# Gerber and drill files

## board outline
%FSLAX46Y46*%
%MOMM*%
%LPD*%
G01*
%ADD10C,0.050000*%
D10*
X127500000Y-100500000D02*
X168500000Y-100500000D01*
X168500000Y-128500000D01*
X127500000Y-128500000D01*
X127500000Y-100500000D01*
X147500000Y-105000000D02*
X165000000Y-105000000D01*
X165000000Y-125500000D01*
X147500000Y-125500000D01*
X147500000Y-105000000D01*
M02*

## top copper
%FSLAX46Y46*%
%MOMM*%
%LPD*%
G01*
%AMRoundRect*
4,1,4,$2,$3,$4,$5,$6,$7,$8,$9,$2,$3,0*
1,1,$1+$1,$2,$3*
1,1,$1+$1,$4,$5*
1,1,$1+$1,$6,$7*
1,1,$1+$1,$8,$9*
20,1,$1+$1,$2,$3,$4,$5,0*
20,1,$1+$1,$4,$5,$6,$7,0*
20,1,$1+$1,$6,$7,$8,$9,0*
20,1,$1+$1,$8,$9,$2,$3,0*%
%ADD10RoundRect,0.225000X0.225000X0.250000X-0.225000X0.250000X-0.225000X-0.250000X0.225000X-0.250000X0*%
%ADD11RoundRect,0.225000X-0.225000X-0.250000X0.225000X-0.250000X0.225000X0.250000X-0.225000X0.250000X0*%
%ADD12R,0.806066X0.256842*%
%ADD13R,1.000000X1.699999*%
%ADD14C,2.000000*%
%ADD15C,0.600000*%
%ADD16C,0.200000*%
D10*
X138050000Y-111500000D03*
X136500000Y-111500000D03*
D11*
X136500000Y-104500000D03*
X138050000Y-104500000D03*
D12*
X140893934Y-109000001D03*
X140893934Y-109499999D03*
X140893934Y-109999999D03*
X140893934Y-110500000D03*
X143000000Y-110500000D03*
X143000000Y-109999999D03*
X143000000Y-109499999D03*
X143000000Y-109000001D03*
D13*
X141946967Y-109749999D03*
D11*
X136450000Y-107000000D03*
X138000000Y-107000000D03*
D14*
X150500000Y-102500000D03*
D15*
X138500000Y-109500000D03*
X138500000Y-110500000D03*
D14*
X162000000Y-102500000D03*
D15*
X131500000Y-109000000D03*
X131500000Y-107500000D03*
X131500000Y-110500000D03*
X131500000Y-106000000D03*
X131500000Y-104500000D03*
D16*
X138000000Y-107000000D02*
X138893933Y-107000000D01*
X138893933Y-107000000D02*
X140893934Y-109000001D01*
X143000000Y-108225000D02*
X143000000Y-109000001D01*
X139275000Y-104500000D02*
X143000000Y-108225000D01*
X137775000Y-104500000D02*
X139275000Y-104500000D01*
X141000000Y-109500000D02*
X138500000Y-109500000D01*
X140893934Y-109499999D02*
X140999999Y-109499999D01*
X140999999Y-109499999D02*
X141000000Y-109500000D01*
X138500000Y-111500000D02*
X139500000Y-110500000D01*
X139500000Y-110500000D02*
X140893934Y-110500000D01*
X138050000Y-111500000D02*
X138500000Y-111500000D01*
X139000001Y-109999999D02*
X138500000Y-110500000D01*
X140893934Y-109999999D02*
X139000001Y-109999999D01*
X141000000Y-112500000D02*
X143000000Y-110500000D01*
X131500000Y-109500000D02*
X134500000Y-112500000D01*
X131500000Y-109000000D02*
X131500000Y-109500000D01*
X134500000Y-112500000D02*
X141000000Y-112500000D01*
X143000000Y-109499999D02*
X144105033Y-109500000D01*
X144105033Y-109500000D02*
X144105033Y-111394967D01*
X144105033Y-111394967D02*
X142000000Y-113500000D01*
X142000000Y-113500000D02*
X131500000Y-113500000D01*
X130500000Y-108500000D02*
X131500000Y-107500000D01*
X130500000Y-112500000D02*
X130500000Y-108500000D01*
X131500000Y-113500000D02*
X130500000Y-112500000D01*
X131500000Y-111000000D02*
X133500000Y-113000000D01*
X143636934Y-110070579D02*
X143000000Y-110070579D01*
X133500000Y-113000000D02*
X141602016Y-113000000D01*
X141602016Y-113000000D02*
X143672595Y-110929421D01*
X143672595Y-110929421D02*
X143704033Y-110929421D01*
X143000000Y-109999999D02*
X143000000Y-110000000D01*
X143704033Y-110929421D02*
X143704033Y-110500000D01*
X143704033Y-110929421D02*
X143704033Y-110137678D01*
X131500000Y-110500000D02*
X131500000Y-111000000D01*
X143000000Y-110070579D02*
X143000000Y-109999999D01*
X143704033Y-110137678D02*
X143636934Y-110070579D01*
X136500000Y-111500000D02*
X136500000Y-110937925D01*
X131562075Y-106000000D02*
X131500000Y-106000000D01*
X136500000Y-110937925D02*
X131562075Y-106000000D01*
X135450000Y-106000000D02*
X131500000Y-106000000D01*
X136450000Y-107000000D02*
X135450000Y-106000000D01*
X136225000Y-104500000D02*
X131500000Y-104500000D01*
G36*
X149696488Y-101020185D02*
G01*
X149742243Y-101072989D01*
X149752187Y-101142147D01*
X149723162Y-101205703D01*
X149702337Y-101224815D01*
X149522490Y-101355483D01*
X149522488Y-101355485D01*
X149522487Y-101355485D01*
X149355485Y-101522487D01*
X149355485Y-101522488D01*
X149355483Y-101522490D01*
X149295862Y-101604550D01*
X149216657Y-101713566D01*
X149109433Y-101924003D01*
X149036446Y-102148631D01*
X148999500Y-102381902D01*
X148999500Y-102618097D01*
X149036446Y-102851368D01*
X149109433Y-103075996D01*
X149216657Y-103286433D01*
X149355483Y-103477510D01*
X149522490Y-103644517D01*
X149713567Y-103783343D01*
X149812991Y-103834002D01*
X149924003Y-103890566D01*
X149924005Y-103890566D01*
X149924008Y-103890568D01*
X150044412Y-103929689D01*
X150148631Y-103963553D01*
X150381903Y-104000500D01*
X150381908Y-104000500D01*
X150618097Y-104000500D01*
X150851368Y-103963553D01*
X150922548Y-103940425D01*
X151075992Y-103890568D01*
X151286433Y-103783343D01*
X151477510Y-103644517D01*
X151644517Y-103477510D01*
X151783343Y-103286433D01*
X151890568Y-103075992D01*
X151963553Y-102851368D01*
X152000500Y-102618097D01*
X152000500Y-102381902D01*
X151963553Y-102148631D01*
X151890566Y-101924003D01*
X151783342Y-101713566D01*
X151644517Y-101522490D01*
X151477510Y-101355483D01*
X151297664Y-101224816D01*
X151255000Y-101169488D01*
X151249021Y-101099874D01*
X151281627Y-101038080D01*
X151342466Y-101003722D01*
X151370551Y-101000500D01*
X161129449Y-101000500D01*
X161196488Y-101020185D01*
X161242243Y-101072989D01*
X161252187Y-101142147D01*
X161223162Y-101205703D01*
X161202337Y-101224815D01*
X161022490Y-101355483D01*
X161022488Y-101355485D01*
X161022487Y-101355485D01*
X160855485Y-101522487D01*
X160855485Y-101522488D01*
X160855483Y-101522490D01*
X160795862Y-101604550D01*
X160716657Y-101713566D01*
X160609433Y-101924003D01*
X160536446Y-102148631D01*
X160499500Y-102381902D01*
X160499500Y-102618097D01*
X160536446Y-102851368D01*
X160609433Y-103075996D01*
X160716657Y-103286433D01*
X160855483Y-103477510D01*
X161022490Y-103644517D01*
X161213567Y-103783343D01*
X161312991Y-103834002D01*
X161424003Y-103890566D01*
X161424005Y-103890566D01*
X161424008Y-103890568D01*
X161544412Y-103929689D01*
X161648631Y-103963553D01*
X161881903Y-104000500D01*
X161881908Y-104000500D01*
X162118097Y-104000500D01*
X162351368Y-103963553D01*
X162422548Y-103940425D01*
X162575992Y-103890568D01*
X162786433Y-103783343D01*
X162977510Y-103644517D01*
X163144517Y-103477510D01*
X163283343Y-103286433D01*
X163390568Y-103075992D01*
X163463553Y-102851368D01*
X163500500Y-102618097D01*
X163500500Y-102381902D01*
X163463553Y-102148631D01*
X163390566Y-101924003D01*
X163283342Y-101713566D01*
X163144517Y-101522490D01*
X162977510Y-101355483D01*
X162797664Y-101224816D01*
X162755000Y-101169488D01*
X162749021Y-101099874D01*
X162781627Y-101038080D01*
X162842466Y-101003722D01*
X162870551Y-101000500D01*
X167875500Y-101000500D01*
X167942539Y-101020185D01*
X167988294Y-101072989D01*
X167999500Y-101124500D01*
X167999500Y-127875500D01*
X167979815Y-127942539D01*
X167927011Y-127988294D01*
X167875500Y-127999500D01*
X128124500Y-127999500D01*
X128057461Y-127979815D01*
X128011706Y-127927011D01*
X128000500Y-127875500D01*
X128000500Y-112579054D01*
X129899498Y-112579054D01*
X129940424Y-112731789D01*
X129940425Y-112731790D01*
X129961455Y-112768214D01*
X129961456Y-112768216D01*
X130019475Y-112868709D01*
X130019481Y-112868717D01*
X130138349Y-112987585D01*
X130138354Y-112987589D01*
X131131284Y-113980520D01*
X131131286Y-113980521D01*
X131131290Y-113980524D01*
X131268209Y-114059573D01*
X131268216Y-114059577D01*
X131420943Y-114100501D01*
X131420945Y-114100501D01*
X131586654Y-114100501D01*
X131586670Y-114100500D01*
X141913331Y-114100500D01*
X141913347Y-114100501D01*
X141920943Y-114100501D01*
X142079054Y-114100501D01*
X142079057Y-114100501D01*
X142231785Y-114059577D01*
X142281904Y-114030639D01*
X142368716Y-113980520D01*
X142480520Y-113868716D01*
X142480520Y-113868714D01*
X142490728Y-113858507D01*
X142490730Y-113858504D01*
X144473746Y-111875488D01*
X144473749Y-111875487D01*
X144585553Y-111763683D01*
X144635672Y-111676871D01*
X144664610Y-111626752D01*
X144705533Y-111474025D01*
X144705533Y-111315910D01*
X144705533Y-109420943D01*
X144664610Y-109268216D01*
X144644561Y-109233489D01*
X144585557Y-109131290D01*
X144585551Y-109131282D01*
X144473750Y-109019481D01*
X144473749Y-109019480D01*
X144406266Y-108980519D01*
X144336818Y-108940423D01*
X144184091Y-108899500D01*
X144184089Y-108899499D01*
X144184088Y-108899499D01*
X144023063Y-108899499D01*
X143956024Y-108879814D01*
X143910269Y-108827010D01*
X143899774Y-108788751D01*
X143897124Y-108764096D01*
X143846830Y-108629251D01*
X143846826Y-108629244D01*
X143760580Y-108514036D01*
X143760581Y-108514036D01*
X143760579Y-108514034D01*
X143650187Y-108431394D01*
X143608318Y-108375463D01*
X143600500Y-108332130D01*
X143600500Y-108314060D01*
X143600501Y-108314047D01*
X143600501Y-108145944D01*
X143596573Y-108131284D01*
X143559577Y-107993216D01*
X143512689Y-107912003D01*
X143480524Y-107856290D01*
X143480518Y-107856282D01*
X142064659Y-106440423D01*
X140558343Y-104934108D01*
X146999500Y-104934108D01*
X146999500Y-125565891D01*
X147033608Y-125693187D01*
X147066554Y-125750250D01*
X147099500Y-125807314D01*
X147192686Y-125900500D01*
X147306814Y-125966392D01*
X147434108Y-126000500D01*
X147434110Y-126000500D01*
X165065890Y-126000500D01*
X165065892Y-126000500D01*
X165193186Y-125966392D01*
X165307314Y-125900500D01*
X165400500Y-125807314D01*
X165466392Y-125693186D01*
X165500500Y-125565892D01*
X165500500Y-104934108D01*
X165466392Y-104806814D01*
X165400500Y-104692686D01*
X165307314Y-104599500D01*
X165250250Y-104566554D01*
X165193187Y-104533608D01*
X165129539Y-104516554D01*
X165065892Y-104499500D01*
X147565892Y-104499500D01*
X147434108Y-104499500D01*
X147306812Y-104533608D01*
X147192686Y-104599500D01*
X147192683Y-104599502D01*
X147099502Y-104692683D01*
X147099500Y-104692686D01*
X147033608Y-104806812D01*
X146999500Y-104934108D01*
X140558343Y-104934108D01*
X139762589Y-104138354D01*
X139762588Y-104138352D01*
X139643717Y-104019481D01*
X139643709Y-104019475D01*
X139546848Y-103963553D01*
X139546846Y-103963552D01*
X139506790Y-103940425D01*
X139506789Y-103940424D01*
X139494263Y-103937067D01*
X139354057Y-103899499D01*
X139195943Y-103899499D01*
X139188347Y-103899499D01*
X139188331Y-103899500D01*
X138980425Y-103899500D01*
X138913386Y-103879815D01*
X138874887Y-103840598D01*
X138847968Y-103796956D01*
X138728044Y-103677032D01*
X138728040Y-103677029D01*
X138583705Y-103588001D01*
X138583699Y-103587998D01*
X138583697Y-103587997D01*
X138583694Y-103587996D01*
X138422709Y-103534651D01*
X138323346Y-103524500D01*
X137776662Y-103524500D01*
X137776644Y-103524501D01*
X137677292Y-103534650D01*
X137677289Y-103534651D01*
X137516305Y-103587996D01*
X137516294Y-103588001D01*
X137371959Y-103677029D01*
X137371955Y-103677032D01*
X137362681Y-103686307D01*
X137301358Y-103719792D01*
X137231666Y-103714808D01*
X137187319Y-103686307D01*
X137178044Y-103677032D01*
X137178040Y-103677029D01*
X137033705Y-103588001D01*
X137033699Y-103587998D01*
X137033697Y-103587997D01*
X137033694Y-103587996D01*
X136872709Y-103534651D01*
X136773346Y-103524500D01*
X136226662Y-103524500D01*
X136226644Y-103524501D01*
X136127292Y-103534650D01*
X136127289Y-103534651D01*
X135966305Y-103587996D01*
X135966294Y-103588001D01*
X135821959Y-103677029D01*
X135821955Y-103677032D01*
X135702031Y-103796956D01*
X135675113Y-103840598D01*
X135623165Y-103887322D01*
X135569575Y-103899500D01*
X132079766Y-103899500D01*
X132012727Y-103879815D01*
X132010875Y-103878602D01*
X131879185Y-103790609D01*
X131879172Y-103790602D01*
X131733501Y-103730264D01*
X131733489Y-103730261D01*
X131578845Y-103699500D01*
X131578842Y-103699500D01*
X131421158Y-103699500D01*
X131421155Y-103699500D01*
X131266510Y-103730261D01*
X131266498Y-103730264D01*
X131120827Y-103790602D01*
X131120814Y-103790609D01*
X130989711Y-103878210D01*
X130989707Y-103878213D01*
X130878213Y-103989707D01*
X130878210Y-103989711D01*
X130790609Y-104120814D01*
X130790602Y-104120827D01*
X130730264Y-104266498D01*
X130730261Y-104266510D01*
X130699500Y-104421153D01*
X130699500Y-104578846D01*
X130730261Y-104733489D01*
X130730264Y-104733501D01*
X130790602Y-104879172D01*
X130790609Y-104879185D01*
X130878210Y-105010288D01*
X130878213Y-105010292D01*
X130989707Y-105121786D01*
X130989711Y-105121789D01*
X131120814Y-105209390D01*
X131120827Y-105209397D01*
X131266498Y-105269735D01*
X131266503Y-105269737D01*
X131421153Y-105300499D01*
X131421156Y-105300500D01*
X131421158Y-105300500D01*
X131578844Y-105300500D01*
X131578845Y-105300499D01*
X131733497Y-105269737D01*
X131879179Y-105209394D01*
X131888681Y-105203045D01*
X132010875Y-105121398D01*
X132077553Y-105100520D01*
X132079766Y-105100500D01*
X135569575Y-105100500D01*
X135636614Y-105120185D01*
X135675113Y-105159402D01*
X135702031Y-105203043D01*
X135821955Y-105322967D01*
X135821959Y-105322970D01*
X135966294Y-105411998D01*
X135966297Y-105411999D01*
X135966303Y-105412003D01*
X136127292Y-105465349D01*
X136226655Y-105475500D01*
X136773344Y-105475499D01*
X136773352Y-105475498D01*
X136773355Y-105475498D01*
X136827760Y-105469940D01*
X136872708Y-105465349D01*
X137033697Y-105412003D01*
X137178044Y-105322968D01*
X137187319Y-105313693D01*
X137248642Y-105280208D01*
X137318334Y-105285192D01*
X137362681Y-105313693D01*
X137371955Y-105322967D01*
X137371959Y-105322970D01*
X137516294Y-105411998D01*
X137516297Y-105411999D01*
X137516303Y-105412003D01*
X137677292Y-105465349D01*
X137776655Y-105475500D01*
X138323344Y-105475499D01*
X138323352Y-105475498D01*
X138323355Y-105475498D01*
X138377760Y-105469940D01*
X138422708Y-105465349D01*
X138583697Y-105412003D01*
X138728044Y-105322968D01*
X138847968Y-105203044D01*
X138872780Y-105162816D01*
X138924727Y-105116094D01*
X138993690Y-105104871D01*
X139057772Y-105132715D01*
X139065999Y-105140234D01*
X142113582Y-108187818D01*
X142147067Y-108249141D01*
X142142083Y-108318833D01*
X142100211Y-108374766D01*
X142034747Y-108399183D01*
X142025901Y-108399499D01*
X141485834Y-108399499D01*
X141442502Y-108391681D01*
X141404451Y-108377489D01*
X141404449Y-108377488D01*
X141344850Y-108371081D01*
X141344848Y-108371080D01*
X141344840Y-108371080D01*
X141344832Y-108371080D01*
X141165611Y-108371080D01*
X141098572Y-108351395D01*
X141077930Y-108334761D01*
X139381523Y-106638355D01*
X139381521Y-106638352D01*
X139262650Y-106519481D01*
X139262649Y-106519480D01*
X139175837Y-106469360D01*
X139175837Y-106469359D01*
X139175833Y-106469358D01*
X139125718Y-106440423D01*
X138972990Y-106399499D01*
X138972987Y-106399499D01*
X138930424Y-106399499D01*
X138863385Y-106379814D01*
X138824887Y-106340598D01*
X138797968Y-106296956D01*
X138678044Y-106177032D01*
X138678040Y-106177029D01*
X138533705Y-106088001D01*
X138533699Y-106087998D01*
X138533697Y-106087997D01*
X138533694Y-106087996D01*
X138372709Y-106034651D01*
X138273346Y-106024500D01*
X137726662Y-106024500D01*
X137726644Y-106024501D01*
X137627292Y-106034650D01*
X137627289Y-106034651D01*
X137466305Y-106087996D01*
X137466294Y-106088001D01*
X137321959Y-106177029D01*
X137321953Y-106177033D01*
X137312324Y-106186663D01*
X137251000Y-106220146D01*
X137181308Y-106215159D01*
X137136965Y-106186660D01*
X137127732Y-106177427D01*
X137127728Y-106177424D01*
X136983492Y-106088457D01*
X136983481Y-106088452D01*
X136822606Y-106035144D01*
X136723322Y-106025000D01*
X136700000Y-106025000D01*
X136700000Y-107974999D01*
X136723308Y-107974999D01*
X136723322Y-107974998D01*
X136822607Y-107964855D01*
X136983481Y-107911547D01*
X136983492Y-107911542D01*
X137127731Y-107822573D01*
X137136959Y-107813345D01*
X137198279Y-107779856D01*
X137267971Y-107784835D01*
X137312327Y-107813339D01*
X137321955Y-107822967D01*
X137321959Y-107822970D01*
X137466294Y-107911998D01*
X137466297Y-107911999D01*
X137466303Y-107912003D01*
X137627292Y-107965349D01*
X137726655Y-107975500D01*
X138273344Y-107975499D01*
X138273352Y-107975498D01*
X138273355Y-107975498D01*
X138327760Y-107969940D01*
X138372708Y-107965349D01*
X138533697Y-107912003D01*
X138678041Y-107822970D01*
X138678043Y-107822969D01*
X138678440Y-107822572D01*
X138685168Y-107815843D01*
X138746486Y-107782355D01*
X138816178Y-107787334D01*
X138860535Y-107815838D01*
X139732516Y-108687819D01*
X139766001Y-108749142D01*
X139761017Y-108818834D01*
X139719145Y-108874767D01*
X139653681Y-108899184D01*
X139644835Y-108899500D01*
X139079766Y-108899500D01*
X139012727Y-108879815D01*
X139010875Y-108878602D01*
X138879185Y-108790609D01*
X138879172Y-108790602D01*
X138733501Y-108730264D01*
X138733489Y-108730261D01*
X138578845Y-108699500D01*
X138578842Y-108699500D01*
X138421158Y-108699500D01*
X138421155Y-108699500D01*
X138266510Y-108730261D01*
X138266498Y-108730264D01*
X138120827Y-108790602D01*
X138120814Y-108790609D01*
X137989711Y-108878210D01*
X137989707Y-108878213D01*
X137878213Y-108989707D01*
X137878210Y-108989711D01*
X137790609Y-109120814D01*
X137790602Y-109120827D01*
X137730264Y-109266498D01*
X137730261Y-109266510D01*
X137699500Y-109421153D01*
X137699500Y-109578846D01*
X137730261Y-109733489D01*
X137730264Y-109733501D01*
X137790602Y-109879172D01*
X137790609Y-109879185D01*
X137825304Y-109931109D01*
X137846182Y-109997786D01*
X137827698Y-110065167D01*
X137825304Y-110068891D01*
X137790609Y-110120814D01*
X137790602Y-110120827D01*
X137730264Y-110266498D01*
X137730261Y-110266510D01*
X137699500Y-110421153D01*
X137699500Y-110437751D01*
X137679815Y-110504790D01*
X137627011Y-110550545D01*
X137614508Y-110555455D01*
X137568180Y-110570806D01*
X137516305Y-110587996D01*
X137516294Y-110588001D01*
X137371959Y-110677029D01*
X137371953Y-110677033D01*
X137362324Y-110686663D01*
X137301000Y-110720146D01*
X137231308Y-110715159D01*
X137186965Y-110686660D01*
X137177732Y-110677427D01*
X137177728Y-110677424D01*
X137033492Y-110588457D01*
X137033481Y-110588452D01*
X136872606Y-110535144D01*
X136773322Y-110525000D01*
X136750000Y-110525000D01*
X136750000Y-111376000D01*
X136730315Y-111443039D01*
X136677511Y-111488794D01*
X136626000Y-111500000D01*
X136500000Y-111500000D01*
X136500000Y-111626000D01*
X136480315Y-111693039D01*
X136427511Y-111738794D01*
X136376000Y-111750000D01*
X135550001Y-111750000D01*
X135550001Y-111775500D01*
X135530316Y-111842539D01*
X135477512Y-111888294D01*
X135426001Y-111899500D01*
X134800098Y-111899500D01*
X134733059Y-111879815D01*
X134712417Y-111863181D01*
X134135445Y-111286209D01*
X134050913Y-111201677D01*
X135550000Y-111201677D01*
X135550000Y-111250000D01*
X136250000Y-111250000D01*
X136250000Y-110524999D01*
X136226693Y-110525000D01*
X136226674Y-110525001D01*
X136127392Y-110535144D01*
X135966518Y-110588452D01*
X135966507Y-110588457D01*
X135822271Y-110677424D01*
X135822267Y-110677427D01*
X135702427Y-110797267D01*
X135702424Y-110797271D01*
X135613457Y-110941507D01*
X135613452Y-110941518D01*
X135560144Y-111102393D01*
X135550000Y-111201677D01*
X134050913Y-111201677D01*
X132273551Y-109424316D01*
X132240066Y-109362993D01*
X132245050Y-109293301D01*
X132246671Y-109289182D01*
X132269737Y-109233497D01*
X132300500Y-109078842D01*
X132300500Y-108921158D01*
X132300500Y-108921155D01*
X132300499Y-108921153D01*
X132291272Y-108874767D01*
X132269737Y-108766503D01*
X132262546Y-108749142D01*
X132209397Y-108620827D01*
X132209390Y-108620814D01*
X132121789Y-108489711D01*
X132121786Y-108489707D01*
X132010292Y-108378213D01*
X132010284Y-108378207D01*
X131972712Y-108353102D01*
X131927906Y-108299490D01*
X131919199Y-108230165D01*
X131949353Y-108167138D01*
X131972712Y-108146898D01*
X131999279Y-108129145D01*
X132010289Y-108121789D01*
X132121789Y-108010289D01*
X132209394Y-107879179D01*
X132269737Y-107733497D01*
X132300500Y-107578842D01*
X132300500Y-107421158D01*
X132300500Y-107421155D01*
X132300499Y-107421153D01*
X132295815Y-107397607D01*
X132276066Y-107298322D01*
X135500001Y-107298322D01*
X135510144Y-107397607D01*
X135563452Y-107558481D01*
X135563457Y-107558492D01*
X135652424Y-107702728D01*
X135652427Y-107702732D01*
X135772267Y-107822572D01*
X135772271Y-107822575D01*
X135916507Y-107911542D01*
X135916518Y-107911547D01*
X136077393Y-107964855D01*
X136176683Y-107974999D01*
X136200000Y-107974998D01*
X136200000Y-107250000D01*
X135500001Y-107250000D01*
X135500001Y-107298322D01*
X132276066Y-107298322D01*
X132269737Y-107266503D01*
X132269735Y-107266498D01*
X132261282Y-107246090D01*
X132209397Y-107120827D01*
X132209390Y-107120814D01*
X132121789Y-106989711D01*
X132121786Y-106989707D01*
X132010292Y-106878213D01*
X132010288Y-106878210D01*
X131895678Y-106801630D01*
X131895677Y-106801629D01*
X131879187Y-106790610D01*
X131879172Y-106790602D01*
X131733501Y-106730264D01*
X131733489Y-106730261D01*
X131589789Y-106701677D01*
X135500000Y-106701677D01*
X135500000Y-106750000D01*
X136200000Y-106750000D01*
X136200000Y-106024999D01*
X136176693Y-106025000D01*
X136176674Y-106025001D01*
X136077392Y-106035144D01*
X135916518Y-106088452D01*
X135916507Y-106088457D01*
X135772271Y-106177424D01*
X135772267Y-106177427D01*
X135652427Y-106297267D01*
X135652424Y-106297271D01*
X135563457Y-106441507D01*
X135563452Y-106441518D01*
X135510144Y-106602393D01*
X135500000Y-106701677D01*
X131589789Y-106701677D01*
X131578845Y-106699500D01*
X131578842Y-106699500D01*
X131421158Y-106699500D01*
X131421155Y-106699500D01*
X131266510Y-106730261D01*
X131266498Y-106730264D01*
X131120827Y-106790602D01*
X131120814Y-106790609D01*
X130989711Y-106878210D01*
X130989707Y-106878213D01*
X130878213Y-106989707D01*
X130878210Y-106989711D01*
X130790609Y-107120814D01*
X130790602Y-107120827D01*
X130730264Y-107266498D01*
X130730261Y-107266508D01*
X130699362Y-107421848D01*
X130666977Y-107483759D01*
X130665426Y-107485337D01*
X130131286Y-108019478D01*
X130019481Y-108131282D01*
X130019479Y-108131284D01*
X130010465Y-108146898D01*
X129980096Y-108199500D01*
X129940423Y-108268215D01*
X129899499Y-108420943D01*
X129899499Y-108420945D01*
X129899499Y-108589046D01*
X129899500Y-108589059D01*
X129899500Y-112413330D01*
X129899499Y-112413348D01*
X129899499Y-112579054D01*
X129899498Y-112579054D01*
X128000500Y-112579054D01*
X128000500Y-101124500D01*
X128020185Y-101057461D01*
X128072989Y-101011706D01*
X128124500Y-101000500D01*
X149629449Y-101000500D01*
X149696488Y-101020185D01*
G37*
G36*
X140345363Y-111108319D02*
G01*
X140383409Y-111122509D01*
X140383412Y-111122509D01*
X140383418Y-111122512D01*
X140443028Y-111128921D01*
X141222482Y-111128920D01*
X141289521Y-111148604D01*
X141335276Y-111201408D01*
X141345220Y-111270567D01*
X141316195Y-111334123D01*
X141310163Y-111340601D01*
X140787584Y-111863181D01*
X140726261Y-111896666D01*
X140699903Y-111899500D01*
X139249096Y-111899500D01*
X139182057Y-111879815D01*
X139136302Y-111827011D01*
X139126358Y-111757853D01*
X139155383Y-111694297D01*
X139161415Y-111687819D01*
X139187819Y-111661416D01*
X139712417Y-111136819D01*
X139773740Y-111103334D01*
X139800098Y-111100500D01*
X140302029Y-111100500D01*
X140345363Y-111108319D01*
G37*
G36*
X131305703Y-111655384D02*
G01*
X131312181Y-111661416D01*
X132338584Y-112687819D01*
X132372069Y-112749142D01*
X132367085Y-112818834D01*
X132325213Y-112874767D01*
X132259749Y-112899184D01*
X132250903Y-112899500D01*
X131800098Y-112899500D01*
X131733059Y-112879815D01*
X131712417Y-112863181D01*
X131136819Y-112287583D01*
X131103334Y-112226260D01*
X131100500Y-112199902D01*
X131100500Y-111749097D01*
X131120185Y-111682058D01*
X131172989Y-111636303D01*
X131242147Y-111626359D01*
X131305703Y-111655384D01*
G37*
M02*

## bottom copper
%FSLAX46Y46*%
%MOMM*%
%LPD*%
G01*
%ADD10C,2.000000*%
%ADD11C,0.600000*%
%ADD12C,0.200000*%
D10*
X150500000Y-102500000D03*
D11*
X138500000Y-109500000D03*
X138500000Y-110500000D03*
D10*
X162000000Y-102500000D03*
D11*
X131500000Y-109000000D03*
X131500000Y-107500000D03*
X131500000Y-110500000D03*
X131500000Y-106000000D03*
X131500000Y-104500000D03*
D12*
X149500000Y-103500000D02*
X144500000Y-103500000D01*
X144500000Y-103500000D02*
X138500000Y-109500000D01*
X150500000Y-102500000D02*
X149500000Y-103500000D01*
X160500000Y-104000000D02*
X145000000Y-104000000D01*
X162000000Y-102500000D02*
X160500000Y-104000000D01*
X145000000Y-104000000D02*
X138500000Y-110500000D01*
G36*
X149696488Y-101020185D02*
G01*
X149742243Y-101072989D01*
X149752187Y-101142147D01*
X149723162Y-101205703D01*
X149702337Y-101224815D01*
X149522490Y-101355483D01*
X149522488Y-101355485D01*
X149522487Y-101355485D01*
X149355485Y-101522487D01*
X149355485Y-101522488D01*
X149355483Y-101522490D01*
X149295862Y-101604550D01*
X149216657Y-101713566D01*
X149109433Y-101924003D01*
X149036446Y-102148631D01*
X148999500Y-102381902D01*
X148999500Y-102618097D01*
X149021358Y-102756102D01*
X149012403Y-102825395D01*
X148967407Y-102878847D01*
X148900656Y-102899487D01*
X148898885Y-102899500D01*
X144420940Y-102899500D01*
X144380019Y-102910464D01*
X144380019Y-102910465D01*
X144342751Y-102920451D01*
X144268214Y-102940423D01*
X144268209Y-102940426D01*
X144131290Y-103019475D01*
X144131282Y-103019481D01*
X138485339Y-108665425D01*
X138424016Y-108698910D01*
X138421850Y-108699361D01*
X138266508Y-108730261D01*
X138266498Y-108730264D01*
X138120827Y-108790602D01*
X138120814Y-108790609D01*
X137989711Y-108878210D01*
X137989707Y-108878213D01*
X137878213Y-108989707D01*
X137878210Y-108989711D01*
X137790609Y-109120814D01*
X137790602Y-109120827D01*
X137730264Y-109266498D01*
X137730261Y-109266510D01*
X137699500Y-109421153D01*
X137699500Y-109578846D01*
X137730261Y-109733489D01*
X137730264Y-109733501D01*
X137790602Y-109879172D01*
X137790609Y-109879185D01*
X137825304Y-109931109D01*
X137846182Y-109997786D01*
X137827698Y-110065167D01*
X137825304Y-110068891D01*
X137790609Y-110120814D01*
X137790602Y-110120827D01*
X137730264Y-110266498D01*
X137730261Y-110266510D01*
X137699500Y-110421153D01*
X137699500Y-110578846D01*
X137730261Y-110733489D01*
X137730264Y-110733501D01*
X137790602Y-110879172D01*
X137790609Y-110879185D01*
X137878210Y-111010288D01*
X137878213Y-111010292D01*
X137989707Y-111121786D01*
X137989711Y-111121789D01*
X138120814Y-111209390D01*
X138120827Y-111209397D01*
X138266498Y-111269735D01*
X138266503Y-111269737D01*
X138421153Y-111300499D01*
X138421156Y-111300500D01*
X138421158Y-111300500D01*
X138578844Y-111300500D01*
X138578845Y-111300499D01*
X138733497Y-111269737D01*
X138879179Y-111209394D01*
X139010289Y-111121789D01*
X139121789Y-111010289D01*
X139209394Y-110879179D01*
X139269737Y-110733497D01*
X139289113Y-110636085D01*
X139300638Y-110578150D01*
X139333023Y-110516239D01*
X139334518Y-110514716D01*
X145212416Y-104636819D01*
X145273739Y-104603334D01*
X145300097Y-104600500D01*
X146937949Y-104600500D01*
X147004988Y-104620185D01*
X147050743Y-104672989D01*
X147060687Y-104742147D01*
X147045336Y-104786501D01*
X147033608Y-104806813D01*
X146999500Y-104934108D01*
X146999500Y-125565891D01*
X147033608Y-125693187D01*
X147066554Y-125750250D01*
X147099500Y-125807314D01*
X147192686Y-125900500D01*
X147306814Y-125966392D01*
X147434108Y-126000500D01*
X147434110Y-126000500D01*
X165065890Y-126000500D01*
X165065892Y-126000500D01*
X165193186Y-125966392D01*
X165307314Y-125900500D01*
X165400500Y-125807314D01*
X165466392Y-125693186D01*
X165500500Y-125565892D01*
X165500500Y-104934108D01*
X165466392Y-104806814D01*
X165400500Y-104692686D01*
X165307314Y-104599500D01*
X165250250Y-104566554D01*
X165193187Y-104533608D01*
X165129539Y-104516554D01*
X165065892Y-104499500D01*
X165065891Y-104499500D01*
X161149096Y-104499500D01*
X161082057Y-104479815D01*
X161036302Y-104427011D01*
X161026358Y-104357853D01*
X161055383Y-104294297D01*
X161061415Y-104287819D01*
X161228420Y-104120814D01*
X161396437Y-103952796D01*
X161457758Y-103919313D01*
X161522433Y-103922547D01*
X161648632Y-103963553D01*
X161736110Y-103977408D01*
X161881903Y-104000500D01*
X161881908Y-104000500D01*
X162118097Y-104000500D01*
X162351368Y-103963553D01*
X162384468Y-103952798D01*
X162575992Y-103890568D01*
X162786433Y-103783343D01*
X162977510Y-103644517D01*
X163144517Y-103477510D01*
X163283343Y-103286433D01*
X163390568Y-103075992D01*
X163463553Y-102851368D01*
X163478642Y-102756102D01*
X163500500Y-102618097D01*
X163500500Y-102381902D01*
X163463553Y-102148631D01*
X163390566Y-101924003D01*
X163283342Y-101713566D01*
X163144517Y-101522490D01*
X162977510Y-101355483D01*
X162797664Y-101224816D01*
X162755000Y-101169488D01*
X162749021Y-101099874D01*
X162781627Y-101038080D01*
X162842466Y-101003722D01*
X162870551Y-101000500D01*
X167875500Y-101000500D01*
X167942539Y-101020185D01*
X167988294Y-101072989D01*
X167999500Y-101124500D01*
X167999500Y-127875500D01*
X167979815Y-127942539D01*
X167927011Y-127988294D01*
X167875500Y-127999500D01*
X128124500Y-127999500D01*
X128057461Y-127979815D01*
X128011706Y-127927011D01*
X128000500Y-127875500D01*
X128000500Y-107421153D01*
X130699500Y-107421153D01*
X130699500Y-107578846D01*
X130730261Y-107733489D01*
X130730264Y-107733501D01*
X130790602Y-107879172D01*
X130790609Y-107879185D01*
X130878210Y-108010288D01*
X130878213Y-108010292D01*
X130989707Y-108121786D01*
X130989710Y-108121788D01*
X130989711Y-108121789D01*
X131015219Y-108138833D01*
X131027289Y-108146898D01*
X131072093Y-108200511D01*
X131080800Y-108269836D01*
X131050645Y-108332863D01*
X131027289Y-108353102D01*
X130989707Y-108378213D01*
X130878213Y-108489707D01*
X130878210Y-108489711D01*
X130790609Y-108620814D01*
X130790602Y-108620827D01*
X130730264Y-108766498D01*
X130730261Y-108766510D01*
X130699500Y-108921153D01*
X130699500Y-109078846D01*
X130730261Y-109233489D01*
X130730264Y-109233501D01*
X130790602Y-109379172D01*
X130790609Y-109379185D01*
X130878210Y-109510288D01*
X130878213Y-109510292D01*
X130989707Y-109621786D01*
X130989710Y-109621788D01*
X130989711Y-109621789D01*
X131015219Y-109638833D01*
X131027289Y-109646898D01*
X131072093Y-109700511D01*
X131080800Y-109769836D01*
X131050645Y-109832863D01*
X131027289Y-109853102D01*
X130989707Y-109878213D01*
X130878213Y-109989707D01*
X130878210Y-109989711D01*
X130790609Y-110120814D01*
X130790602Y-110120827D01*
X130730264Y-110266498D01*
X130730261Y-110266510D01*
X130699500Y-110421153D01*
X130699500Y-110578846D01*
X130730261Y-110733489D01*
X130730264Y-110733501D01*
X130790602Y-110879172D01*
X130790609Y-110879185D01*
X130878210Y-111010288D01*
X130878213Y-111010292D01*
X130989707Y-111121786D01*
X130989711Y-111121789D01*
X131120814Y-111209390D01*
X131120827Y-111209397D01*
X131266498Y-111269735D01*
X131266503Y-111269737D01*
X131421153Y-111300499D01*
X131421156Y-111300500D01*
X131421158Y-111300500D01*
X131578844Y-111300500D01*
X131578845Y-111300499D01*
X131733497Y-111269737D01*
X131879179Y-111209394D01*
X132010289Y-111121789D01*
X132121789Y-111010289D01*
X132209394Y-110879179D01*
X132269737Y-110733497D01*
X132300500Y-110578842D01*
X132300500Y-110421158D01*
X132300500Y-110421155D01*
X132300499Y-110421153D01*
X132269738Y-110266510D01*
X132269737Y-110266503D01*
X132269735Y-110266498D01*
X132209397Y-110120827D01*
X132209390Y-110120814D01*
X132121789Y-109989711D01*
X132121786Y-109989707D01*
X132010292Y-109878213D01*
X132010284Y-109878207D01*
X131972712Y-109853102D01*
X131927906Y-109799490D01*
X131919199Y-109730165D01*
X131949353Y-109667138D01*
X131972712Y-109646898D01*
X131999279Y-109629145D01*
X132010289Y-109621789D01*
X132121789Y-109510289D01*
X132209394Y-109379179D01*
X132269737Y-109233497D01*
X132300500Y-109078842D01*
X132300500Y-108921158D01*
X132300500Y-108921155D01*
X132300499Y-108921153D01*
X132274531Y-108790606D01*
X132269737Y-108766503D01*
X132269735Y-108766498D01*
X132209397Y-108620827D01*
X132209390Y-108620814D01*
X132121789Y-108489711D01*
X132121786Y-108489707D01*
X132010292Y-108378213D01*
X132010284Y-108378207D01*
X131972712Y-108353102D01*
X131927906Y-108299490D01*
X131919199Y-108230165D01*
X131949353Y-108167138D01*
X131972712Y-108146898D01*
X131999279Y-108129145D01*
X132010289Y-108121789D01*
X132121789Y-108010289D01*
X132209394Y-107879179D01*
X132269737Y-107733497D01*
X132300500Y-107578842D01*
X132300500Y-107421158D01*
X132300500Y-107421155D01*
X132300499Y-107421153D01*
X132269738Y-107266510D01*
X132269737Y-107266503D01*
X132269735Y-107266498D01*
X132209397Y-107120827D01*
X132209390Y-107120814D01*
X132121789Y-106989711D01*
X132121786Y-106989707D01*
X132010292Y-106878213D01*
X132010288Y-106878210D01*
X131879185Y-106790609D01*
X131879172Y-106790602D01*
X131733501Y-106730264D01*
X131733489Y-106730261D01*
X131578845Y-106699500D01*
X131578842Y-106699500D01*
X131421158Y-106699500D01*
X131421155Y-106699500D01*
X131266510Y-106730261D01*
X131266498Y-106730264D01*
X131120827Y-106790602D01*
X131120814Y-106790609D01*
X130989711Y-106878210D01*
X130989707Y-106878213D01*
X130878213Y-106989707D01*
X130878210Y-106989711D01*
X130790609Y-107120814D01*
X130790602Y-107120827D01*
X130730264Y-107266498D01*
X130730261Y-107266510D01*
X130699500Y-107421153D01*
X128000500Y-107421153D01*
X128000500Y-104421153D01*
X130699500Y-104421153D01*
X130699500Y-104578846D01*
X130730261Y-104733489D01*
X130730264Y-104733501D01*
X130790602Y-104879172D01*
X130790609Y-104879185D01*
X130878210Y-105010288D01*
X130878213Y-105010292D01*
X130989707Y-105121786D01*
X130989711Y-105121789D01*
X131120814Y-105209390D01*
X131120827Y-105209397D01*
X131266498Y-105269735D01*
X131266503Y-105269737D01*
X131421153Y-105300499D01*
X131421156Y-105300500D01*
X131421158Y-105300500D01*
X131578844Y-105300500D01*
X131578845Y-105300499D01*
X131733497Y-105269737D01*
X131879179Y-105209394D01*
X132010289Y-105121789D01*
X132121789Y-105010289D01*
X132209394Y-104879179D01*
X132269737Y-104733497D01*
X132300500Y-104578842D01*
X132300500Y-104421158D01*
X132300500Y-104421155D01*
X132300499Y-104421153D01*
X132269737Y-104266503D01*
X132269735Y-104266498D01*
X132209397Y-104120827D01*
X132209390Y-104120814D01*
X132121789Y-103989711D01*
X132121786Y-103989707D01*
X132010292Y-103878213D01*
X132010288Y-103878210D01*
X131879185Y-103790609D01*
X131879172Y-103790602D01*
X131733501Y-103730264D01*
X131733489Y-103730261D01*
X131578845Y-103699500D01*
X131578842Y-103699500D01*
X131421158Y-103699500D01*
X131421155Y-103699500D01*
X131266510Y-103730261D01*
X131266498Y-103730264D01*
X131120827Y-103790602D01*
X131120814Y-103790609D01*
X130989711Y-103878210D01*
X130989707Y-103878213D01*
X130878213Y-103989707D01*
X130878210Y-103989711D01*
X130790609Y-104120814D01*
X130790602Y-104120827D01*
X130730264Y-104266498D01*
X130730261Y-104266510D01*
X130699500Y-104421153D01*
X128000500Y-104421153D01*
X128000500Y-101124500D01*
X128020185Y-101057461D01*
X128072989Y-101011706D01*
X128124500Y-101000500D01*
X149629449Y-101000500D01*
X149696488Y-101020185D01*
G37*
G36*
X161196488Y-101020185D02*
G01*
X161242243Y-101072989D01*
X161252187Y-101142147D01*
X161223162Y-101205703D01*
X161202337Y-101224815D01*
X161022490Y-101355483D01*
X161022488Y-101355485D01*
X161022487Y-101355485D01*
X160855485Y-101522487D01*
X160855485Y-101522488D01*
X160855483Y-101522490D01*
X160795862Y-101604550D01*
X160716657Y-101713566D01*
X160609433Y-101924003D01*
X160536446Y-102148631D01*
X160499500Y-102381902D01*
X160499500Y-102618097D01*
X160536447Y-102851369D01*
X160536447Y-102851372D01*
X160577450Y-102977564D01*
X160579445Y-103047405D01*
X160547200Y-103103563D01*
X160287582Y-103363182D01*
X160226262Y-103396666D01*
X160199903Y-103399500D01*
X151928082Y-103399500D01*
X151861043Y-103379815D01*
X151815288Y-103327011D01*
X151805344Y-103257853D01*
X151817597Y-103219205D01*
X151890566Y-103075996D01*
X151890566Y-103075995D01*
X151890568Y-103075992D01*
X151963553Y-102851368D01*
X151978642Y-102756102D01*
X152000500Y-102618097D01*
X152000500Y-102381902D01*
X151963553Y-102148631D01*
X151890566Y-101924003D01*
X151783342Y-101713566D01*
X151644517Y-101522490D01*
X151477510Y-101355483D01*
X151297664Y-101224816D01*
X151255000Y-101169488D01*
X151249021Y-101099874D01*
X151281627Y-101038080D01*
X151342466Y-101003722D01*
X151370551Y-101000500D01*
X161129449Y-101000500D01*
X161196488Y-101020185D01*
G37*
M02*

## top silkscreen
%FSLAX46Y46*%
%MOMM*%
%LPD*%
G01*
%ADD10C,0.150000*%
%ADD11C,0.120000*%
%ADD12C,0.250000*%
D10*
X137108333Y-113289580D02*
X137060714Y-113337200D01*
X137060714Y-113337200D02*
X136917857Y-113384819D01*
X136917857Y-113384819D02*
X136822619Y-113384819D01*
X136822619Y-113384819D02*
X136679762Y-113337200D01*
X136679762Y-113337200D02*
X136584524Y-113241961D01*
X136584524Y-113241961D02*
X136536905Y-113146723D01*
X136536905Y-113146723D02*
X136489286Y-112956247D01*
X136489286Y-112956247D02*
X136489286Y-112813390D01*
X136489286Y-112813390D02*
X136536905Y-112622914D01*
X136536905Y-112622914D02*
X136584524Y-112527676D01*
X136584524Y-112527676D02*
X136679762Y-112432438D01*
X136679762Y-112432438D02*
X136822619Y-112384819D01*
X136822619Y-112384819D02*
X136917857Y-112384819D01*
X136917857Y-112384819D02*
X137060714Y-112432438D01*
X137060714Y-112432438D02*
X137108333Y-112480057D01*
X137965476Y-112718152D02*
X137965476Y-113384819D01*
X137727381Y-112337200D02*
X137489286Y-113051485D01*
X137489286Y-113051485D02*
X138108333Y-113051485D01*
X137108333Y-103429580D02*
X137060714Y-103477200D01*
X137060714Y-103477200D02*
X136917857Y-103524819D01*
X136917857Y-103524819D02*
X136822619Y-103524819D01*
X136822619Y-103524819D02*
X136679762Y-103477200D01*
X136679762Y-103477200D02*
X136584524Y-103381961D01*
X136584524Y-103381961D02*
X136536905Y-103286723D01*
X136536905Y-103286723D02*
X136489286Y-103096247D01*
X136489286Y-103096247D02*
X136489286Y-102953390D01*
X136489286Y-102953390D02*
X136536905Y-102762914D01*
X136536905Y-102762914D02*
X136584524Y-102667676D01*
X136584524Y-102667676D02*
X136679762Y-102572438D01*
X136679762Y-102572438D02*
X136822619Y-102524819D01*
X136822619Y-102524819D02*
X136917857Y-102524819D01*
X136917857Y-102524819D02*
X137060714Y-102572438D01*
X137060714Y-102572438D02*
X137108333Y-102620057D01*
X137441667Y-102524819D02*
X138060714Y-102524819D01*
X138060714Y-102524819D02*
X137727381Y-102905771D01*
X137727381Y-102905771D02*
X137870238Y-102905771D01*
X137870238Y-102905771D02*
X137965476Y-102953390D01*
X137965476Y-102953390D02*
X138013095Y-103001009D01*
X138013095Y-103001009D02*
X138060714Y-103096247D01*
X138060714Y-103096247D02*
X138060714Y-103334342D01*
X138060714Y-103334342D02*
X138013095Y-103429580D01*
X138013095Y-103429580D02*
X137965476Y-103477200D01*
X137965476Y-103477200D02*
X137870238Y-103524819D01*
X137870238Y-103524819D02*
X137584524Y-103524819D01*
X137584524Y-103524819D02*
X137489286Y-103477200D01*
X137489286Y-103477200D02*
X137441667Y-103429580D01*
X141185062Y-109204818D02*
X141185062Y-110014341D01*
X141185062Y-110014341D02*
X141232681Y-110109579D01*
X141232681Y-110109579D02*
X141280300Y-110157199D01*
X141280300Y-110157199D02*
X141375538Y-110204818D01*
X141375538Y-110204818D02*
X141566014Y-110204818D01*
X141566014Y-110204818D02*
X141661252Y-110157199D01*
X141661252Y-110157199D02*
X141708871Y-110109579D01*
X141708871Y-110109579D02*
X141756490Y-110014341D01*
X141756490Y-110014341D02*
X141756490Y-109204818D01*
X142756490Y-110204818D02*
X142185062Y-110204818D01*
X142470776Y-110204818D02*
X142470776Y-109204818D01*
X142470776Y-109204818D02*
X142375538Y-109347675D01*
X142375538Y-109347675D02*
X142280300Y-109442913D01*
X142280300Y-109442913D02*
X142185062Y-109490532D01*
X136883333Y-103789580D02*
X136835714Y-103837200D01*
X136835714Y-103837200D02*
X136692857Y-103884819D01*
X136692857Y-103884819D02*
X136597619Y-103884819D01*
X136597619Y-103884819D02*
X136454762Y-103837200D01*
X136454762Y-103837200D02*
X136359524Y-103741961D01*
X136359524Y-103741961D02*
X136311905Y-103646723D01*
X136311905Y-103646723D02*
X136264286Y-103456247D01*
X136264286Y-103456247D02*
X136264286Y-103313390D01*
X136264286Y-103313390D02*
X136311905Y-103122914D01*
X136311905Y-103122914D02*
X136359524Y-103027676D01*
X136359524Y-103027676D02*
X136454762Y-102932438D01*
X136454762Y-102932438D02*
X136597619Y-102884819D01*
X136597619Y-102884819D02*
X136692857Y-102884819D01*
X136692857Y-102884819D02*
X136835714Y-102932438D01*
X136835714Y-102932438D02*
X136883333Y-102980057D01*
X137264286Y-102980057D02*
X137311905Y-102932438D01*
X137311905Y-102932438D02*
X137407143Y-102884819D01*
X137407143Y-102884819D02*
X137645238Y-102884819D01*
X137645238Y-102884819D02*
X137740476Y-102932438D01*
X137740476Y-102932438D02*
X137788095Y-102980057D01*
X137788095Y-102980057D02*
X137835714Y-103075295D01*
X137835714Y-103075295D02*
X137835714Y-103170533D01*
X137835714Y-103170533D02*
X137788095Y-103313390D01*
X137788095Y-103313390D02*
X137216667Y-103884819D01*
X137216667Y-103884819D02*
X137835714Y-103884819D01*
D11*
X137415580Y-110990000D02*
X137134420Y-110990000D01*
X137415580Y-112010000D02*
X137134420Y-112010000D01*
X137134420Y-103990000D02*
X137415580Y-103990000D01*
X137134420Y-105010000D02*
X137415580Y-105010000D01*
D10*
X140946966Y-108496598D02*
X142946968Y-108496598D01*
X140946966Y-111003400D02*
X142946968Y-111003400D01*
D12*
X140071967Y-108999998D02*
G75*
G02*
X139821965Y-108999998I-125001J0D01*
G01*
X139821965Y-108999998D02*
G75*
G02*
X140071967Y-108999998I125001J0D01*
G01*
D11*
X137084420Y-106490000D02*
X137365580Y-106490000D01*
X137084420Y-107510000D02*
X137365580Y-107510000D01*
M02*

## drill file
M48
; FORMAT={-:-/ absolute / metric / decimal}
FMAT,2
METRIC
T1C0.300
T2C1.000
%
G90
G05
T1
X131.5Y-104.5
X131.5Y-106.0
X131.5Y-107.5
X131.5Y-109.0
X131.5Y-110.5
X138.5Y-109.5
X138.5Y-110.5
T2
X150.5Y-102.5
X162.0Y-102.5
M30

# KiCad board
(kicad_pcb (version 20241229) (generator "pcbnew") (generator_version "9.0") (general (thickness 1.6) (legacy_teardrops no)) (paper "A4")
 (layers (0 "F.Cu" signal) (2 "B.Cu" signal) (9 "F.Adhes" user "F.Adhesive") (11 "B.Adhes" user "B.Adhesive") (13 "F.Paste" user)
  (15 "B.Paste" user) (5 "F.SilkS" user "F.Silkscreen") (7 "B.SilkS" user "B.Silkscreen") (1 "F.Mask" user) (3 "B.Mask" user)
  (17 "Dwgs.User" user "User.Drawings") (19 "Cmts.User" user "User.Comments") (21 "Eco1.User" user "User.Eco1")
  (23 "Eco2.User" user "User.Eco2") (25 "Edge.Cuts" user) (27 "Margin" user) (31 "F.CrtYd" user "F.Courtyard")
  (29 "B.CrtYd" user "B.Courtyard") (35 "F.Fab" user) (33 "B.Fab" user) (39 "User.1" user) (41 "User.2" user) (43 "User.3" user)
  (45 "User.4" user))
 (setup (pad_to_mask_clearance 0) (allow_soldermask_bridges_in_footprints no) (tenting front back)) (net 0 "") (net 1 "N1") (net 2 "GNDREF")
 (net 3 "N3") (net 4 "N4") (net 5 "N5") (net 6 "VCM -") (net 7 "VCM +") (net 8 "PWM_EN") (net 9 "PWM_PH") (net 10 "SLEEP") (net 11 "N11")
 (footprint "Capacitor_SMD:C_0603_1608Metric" (layer "F.Cu") (at 137.275 111.5 180)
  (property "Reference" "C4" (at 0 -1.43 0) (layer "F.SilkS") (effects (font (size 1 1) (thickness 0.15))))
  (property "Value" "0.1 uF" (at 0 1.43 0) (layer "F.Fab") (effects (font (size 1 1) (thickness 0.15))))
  (fp_line (start -0.14058 0.51) (end 0.14058 0.51) (stroke (width 0.12) (type solid)) (layer "F.SilkS"))
  (fp_line (start -0.14058 -0.51) (end 0.14058 -0.51) (stroke (width 0.12) (type solid)) (layer "F.SilkS"))
  (pad "1" smd roundrect (at -0.775 0 180) (size 0.9 0.95) (layers "F.Cu" "F.Mask" "F.Paste") (roundrect_rratio 0.25) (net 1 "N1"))
  (pad "2" smd roundrect (at 0.775 0 180) (size 0.9 0.95) (layers "F.Cu" "F.Mask" "F.Paste") (roundrect_rratio 0.25) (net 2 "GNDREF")))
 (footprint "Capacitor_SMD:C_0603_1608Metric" (layer "F.Cu") (at 137.275 104.5)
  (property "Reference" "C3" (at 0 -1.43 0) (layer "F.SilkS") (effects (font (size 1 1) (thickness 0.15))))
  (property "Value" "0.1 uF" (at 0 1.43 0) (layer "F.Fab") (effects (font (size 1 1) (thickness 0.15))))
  (fp_line (start -0.14058 -0.51) (end 0.14058 -0.51) (stroke (width 0.12) (type solid)) (layer "F.SilkS"))
  (fp_line (start -0.14058 0.51) (end 0.14058 0.51) (stroke (width 0.12) (type solid)) (layer "F.SilkS"))
  (pad "1" smd roundrect (at -0.775 0) (size 0.9 0.95) (layers "F.Cu" "F.Mask" "F.Paste") (roundrect_rratio 0.25) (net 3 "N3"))
  (pad "2" smd roundrect (at 0.775 0) (size 0.9 0.95) (layers "F.Cu" "F.Mask" "F.Paste") (roundrect_rratio 0.25) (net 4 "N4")))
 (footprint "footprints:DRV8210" (layer "F.Cu") (at 141.946967 109.749999)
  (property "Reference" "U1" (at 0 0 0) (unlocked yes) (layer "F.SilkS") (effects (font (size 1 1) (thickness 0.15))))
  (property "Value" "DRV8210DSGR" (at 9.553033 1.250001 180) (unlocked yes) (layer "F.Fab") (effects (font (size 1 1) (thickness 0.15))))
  (fp_line (start -1.000001 -1.253401) (end 1.000001 -1.253401) (stroke (width 0.15) (type solid)) (layer "F.SilkS"))
  (fp_line (start -1.000001 1.253401) (end 1.000001 1.253401) (stroke (width 0.15) (type solid)) (layer "F.SilkS"))
  (fp_circle (center -2.000001 -0.750001) (end -1.875 -0.750001) (stroke (width 0.25) (type solid)) (fill no) (layer "F.SilkS"))
  (pad "1" smd rect (at -1.053033 -0.749998) (size 0.806066 0.256842) (layers "F.Cu" "F.Mask" "F.Paste") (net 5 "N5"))
  (pad "2" smd rect (at -1.053033 -0.25) (size 0.806066 0.256842) (layers "F.Cu" "F.Mask" "F.Paste") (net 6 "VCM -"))
  (pad "3" smd rect (at -1.053033 0.25) (size 0.806066 0.256842) (layers "F.Cu" "F.Mask" "F.Paste") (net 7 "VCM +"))
  (pad "4" smd rect (at -1.053033 0.750001) (size 0.806066 0.256842) (layers "F.Cu" "F.Mask" "F.Paste") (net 1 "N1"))
  (pad "5" smd rect (at 1.053033 0.750001) (size 0.806066 0.256842) (layers "F.Cu" "F.Mask" "F.Paste") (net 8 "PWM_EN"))
  (pad "6" smd rect (at 1.053033 0.25) (size 0.806066 0.256842) (layers "F.Cu" "F.Mask" "F.Paste") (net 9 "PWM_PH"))
  (pad "7" smd rect (at 1.053033 -0.25) (size 0.806066 0.256842) (layers "F.Cu" "F.Mask" "F.Paste") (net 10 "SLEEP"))
  (pad "8" smd rect (at 1.053033 -0.749998) (size 0.806066 0.256842) (layers "F.Cu" "F.Mask" "F.Paste") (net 4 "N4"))
  (pad "9" smd rect (at 0 0) (size 1 1.699999) (layers "F.Cu" "F.Mask") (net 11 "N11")))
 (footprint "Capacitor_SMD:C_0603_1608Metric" (layer "F.Cu") (at 137.225 107)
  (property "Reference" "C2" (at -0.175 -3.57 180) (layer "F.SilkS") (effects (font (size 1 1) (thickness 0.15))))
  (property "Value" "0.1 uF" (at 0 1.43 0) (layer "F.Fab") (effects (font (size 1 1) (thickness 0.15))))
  (fp_line (start -0.14058 -0.51) (end 0.14058 -0.51) (stroke (width 0.12) (type solid)) (layer "F.SilkS"))
  (fp_line (start -0.14058 0.51) (end 0.14058 0.51) (stroke (width 0.12) (type solid)) (layer "F.SilkS"))
  (pad "1" smd roundrect (at -0.775 0) (size 0.9 0.95) (layers "F.Cu" "F.Mask" "F.Paste") (roundrect_rratio 0.25) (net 2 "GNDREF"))
  (pad "2" smd roundrect (at 0.775 0) (size 0.9 0.95) (layers "F.Cu" "F.Mask" "F.Paste") (roundrect_rratio 0.25) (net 5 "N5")))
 (gr_rect (start 127.5 100.5) (end 168.5 128.5) (stroke (width 0.05) (type default)) (fill no) (layer "Edge.Cuts"))
 (gr_rect (start 147.5 105) (end 165 125.5) (stroke (width 0.05) (type default)) (fill no) (layer "Edge.Cuts"))
 (segment (start 138 107) (end 138.893933 107) (width 0.2) (layer "F.Cu") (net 5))
 (segment (start 138.893933 107) (end 140.893934 109.000001) (width 0.2) (layer "F.Cu") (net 5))
 (segment (start 143 108.225) (end 143 109.000001) (width 0.2) (layer "F.Cu") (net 4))
 (segment (start 139.275 104.5) (end 143 108.225) (width 0.2) (layer "F.Cu") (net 4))
 (segment (start 137.775 104.5) (end 139.275 104.5) (width 0.2) (layer "F.Cu") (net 4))
 (segment (start 141 109.5) (end 138.5 109.5) (width 0.2) (layer "F.Cu") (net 6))
 (segment (start 140.893934 109.499999) (end 140.999999 109.499999) (width 0.2) (layer "F.Cu") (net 6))
 (segment (start 140.999999 109.499999) (end 141 109.5) (width 0.2) (layer "F.Cu") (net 6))
 (via (at 150.5 102.5) (size 2) (drill 1) (layers "F.Cu" "B.Cu") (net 6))
 (via (at 138.5 109.5) (size 0.6) (drill 0.3) (layers "F.Cu" "B.Cu") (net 6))
 (segment (start 149.5 103.5) (end 144.5 103.5) (width 0.2) (layer "B.Cu") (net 6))
 (segment (start 144.5 103.5) (end 138.5 109.5) (width 0.2) (layer "B.Cu") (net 6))
 (segment (start 150.5 102.5) (end 149.5 103.5) (width 0.2) (layer "B.Cu") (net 6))
 (segment (start 138.5 111.5) (end 139.5 110.5) (width 0.2) (layer "F.Cu") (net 1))
 (segment (start 139.5 110.5) (end 140.893934 110.5) (width 0.2) (layer "F.Cu") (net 1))
 (segment (start 138.05 111.5) (end 138.5 111.5) (width 0.2) (layer "F.Cu") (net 1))
 (segment (start 139.000001 109.999999) (end 138.5 110.5) (width 0.2) (layer "F.Cu") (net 7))
 (segment (start 140.893934 109.999999) (end 139.000001 109.999999) (width 0.2) (layer "F.Cu") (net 7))
 (via (at 138.5 110.5) (size 0.6) (drill 0.3) (layers "F.Cu" "B.Cu") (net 7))
 (via (at 162 102.5) (size 2) (drill 1) (layers "F.Cu" "B.Cu") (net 7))
 (segment (start 160.5 104) (end 145 104) (width 0.2) (layer "B.Cu") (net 7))
 (segment (start 162 102.5) (end 160.5 104) (width 0.2) (layer "B.Cu") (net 7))
 (segment (start 145 104) (end 138.5 110.5) (width 0.2) (layer "B.Cu") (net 7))
 (segment (start 141 112.5) (end 143 110.5) (width 0.2) (layer "F.Cu") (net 8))
 (segment (start 131.5 109.5) (end 134.5 112.5) (width 0.2) (layer "F.Cu") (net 8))
 (segment (start 131.5 109) (end 131.5 109.5) (width 0.2) (layer "F.Cu") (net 8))
 (segment (start 134.5 112.5) (end 141 112.5) (width 0.2) (layer "F.Cu") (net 8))
 (via (at 131.5 109) (size 0.6) (drill 0.3) (layers "F.Cu" "B.Cu") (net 8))
 (segment (start 143 109.499999) (end 144.105033 109.5) (width 0.2) (layer "F.Cu") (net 10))
 (segment (start 144.105033 109.5) (end 144.105033 111.394967) (width 0.2) (layer "F.Cu") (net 10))
 (segment (start 144.105033 111.394967) (end 142 113.5) (width 0.2) (layer "F.Cu") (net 10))
 (segment (start 142 113.5) (end 131.5 113.5) (width 0.2) (layer "F.Cu") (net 10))
 (segment (start 130.5 108.5) (end 131.5 107.5) (width 0.2) (layer "F.Cu") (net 10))
 (segment (start 130.5 112.5) (end 130.5 108.5) (width 0.2) (layer "F.Cu") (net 10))
 (segment (start 131.5 113.5) (end 130.5 112.5) (width 0.2) (layer "F.Cu") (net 10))
 (via (at 131.5 107.5) (size 0.6) (drill 0.3) (layers "F.Cu" "B.Cu") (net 10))
 (segment (start 131.5 111) (end 133.5 113) (width 0.2) (layer "F.Cu") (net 9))
 (segment (start 143.636934 110.070579) (end 143 110.070579) (width 0.2) (layer "F.Cu") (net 9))
 (segment (start 133.5 113) (end 141.602016 113) (width 0.2) (layer "F.Cu") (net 9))
 (segment (start 141.602016 113) (end 143.672595 110.929421) (width 0.2) (layer "F.Cu") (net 9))
 (segment (start 143.672595 110.929421) (end 143.704033 110.929421) (width 0.2) (layer "F.Cu") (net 9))
 (segment (start 143 109.999999) (end 143 110) (width 0.2) (layer "F.Cu") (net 9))
 (segment (start 143.704033 110.929421) (end 143.704033 110.5) (width 0.2) (layer "F.Cu") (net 9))
 (segment (start 143.704033 110.929421) (end 143.704033 110.137678) (width 0.2) (layer "F.Cu") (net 9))
 (segment (start 131.5 110.5) (end 131.5 111) (width 0.2) (layer "F.Cu") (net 9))
 (segment (start 143 110.070579) (end 143 109.999999) (width 0.2) (layer "F.Cu") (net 9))
 (segment (start 143.704033 110.137678) (end 143.636934 110.070579) (width 0.2) (layer "F.Cu") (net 9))
 (via (at 131.5 110.5) (size 0.6) (drill 0.3) (layers "F.Cu" "B.Cu") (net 9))
 (segment (start 136.5 111.5) (end 136.5 110.937925) (width 0.2) (layer "F.Cu") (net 2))
 (segment (start 131.562075 106) (end 131.5 106) (width 0.2) (layer "F.Cu") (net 2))
 (segment (start 136.5 110.937925) (end 131.562075 106) (width 0.2) (layer "F.Cu") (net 2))
 (segment (start 135.45 106) (end 131.5 106) (width 0.2) (layer "F.Cu") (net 2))
 (segment (start 136.45 107) (end 135.45 106) (width 0.2) (layer "F.Cu") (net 2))
 (via (at 131.5 106) (size 0.6) (drill 0.3) (layers "F.Cu" "B.Cu") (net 2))
 (segment (start 136.225 104.5) (end 131.5 104.5) (width 0.2) (layer "F.Cu") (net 3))
 (via (at 131.5 104.5) (size 0.6) (drill 0.3) (layers "F.Cu" "B.Cu") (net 3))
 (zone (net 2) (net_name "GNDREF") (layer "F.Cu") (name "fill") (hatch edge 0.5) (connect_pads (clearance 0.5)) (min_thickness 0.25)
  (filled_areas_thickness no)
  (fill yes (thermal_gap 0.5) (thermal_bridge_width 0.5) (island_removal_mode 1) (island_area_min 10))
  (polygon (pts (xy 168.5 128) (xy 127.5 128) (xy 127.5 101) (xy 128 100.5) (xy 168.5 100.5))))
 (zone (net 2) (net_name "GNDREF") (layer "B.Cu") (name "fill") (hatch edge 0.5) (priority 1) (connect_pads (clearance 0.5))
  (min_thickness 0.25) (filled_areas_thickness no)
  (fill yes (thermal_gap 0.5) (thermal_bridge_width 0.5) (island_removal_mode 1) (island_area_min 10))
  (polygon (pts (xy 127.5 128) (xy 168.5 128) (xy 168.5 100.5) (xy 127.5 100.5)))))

